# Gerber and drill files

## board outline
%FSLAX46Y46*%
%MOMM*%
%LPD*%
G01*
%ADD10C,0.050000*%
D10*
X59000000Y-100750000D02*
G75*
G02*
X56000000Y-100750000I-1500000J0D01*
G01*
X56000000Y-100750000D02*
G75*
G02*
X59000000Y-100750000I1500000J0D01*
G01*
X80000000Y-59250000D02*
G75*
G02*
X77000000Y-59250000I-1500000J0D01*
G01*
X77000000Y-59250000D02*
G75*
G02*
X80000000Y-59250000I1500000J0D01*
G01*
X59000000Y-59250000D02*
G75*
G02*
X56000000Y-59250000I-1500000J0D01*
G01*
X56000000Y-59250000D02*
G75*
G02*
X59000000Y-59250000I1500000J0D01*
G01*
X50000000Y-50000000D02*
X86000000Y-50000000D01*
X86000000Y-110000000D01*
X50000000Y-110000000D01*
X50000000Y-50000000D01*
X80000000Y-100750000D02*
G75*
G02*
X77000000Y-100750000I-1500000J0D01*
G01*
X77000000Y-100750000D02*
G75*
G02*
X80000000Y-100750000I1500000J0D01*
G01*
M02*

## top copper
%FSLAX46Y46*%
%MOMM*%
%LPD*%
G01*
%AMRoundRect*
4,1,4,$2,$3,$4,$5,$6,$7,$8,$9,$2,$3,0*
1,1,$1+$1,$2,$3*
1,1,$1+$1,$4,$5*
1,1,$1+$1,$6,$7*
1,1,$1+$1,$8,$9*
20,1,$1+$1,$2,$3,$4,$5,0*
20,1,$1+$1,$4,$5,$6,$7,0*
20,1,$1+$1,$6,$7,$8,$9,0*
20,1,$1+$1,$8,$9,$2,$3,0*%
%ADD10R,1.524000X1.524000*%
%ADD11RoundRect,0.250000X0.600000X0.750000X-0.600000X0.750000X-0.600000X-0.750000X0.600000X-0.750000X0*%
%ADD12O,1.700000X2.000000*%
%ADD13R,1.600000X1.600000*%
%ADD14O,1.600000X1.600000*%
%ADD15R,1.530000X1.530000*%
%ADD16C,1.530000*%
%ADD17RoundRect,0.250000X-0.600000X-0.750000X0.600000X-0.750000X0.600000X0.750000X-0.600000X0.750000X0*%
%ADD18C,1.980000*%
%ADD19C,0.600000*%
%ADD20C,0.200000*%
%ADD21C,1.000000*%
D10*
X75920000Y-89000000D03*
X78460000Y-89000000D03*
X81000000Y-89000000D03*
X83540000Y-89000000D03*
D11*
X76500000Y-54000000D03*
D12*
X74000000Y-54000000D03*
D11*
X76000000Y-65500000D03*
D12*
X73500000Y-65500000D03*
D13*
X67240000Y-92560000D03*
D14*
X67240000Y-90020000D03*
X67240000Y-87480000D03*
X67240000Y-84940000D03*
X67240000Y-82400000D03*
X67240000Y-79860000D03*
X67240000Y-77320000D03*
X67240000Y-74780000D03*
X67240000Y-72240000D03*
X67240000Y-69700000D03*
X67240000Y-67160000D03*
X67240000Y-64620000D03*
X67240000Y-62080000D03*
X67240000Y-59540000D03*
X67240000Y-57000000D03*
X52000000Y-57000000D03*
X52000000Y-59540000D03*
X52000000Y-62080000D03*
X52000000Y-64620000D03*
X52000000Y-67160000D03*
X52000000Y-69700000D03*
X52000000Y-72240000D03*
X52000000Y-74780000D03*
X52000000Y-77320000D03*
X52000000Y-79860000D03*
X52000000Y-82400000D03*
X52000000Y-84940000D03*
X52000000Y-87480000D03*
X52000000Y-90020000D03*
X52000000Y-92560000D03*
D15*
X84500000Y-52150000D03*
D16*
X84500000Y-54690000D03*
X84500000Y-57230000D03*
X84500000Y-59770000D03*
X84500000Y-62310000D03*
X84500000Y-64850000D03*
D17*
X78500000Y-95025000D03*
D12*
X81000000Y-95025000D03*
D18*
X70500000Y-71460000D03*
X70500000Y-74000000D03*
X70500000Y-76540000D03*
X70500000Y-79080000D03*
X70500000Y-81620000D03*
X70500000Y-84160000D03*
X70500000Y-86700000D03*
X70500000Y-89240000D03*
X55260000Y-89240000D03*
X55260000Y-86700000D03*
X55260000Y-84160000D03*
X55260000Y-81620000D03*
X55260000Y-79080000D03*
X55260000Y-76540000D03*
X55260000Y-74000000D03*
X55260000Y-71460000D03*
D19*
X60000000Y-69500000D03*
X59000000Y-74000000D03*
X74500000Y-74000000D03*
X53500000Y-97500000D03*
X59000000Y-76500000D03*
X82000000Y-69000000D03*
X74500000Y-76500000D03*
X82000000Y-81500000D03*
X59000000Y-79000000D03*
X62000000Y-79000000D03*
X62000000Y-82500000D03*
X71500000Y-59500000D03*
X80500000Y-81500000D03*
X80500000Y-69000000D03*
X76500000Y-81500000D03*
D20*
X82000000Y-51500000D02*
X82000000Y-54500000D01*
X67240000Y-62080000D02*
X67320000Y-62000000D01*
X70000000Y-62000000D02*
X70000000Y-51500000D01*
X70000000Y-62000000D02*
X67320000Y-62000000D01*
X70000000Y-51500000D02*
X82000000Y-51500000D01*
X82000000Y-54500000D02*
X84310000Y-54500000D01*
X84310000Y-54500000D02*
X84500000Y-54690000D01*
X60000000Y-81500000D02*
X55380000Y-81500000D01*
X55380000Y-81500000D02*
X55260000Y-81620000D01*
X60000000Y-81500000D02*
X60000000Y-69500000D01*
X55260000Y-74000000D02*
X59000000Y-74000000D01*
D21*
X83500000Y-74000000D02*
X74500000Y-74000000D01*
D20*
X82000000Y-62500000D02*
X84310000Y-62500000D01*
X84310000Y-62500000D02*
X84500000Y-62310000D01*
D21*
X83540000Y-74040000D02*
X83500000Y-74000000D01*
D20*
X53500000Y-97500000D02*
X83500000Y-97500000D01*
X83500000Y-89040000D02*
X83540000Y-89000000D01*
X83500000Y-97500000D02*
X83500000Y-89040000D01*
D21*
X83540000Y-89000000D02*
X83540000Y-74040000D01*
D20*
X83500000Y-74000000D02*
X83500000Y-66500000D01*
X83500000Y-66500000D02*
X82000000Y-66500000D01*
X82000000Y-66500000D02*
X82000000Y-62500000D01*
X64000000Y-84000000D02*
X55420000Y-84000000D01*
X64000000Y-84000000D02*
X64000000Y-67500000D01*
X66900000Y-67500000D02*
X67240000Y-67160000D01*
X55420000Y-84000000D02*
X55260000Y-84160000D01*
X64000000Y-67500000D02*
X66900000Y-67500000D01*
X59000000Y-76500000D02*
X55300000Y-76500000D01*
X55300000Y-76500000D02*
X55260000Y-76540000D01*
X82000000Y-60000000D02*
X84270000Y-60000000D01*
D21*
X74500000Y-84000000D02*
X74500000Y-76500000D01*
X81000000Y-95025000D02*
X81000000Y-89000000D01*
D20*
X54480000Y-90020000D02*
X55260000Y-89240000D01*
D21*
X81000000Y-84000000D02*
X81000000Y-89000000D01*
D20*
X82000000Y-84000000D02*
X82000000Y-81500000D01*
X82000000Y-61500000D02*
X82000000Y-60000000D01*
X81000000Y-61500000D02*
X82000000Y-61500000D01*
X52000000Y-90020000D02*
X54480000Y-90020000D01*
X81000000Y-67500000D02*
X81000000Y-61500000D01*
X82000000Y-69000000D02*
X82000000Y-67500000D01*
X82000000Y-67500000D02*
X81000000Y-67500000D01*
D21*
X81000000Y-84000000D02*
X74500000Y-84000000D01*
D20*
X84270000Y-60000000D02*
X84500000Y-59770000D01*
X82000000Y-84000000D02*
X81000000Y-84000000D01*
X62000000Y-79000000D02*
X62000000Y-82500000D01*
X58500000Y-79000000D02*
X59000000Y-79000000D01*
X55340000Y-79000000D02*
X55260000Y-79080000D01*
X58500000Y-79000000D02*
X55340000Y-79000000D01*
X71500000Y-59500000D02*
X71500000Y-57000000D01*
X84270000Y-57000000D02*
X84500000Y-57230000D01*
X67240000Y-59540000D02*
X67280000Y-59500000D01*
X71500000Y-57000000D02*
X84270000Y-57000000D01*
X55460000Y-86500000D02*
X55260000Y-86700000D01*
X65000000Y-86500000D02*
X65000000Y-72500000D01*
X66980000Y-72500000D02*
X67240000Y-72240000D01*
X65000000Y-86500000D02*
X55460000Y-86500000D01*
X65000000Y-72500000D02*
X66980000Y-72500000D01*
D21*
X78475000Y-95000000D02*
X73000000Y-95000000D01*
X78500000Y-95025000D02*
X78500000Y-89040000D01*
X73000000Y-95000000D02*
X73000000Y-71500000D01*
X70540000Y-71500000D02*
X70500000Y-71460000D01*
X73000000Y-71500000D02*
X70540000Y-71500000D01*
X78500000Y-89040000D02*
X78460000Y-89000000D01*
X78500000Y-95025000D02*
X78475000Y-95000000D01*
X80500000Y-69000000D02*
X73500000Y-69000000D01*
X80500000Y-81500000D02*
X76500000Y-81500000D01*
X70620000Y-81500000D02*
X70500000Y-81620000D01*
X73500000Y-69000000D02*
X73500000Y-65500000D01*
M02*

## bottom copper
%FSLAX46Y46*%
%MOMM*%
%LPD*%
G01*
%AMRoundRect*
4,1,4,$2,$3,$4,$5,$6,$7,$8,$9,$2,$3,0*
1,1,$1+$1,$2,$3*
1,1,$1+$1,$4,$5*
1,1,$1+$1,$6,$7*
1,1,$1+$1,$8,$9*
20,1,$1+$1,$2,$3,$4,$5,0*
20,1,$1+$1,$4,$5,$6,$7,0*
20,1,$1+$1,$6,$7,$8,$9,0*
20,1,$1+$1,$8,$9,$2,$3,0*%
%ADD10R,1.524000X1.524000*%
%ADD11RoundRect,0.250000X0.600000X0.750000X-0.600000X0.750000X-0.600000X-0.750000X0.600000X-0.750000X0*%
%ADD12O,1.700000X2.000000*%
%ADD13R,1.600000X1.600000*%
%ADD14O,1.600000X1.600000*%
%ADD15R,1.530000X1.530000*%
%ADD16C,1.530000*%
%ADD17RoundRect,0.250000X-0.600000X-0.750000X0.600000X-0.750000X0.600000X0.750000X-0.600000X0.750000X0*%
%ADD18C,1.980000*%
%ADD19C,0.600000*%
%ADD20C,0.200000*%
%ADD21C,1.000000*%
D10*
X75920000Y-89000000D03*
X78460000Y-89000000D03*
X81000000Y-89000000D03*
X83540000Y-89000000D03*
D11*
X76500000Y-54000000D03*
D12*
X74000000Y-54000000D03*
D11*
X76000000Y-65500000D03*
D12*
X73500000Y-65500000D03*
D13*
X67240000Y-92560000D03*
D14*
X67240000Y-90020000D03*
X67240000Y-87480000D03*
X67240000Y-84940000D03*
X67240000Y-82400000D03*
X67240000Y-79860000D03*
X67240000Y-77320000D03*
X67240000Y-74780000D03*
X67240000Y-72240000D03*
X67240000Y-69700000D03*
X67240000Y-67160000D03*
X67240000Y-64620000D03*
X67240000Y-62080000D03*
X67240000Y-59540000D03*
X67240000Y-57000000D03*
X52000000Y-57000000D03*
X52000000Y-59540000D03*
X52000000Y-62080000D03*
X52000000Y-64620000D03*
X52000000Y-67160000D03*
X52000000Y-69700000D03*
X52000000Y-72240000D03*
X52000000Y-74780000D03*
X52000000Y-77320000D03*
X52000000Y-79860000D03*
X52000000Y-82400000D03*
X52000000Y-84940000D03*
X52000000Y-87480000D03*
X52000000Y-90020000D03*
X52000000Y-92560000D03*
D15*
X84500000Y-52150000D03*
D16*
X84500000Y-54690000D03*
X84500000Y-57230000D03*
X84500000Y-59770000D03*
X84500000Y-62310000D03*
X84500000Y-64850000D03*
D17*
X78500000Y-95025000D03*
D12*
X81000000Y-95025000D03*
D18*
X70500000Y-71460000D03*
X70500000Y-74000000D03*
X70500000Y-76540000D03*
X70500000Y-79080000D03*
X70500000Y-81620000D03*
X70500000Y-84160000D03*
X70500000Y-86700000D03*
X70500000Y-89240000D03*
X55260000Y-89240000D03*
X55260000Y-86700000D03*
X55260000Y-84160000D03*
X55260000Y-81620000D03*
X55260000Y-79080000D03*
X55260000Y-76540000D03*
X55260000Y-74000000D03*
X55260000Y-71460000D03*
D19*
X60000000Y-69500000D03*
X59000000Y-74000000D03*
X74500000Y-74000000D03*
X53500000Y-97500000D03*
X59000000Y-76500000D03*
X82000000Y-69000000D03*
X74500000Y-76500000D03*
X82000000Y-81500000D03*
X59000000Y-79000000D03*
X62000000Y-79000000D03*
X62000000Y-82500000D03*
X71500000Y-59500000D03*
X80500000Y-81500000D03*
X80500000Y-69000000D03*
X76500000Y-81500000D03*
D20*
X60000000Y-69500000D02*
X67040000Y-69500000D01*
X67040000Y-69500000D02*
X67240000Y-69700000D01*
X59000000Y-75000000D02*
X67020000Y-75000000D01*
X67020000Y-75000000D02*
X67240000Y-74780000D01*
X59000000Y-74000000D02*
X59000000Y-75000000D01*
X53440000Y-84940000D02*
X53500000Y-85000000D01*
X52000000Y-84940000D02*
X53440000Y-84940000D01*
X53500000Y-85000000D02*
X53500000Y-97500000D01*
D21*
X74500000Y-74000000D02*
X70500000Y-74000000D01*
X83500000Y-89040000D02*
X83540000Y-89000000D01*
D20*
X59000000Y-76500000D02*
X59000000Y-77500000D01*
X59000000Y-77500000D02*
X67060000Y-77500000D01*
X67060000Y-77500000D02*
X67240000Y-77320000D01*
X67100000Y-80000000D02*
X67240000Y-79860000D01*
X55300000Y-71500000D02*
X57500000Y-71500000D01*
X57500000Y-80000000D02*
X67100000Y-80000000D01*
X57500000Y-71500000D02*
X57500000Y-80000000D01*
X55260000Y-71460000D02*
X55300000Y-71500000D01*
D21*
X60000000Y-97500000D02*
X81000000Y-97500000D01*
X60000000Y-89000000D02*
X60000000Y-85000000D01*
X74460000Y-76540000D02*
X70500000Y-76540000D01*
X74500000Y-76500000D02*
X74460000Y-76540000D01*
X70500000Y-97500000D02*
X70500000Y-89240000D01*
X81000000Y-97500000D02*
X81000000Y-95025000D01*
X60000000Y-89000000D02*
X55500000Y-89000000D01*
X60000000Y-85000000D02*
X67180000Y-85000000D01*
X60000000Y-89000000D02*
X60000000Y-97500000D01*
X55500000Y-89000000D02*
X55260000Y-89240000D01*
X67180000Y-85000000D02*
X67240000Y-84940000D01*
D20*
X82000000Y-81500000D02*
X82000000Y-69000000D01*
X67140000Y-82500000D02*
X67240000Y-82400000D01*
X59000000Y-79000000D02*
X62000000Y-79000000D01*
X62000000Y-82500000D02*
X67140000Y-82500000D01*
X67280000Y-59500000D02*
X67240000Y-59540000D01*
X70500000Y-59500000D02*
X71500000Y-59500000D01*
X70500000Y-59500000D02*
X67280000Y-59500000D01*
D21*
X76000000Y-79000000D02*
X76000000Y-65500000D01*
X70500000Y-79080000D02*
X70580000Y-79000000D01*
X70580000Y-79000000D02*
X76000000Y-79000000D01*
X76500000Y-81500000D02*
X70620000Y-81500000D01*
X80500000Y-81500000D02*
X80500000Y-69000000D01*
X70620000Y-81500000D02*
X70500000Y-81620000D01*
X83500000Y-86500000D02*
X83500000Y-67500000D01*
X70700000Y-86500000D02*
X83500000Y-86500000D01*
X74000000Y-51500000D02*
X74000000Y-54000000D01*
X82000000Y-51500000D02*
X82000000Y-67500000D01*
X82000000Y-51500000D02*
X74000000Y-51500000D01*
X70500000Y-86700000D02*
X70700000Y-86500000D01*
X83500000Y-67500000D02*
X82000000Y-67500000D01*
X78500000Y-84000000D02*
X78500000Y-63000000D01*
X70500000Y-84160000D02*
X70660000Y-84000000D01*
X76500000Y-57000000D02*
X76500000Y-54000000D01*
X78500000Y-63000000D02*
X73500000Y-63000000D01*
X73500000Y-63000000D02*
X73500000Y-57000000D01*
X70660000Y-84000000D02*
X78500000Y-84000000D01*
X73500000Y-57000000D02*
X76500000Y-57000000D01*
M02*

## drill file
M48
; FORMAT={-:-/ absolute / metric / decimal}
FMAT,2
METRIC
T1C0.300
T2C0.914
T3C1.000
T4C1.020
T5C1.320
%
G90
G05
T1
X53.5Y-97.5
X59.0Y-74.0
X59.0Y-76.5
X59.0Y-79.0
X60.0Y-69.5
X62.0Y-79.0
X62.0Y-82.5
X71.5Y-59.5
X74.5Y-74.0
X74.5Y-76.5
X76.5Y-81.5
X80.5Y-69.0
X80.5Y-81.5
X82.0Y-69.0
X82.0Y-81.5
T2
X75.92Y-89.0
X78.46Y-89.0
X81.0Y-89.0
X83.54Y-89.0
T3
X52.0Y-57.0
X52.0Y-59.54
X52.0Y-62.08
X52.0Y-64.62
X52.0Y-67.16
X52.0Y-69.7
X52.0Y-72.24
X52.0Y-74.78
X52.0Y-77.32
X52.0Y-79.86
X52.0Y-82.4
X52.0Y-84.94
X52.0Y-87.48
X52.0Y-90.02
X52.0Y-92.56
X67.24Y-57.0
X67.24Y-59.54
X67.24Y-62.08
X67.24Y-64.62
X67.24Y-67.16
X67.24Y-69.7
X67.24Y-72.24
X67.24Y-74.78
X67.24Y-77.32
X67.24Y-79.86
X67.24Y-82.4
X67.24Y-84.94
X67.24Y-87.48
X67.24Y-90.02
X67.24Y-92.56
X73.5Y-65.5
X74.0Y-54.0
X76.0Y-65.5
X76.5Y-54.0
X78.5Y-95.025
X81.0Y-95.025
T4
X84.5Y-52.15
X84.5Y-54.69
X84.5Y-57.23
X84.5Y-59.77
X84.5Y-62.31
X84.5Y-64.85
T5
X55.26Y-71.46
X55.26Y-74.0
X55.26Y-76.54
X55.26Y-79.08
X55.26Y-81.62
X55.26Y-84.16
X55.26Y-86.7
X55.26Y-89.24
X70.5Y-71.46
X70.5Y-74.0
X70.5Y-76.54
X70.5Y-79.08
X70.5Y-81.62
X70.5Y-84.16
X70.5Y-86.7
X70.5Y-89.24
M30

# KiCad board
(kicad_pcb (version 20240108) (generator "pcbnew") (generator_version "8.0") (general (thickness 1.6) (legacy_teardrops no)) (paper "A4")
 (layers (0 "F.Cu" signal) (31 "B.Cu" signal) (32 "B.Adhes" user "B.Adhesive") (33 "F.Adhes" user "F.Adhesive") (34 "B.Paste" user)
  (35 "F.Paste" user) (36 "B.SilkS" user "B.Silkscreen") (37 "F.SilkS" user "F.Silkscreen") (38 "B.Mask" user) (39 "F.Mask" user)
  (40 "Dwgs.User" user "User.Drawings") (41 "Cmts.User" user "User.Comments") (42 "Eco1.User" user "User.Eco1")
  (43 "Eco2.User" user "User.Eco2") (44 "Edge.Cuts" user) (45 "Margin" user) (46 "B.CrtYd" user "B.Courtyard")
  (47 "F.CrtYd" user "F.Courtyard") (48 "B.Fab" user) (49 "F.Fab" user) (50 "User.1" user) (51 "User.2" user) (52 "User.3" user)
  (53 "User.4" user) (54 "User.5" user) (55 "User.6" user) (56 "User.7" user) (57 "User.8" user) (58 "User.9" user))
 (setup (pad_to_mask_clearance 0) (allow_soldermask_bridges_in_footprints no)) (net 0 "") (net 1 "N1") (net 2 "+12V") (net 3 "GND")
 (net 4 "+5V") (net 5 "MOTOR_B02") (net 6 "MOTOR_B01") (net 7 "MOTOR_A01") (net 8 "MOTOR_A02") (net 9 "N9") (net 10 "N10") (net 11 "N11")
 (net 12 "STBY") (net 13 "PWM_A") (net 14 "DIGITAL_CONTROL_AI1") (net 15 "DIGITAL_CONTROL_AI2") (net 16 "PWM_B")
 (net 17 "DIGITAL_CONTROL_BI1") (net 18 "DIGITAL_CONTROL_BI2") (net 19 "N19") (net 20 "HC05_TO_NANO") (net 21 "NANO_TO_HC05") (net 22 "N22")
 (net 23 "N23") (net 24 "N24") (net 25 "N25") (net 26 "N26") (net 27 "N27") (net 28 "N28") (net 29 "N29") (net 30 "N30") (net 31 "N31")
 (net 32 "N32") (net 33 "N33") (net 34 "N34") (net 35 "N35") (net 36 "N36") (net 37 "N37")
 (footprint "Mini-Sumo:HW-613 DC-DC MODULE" (layer "F.Cu") (at 75.92 89 90)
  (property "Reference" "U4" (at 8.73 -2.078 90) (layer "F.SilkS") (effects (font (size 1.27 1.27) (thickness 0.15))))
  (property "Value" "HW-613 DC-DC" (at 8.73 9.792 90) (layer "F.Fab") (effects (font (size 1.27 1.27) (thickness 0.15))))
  (pad "1" thru_hole rect (at 0 0 90) (size 1.524 1.524) (drill 0.9144) (layers "*.Cu" "*.Mask") (remove_unused_layers no) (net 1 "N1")
   (solder_mask_margin 0.0508) (thermal_bridge_angle 0))
  (pad "2" thru_hole rect (at 0 2.54 90) (size 1.524 1.524) (drill 0.9144) (layers "*.Cu" "*.Mask") (remove_unused_layers no) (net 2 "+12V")
   (solder_mask_margin 0.0508) (thermal_bridge_angle 0))
  (pad "3" thru_hole rect (at 0 5.08 90) (size 1.524 1.524) (drill 0.9144) (layers "*.Cu" "*.Mask") (remove_unused_layers no) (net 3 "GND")
   (solder_mask_margin 0.0508) (thermal_bridge_angle 0))
  (pad "4" thru_hole rect (at 0 7.62 90) (size 1.524 1.524) (drill 0.9144) (layers "*.Cu" "*.Mask") (remove_unused_layers no) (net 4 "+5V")
   (solder_mask_margin 0.0508) (thermal_bridge_angle 0)))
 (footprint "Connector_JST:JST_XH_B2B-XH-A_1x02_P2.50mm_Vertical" (layer "F.Cu") (at 76.5 54 180)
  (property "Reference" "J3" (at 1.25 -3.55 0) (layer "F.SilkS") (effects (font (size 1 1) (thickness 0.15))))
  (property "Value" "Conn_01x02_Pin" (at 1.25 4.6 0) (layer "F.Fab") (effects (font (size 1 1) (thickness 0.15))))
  (pad "1" thru_hole roundrect (at 0 0 180) (size 1.7 2) (drill 1) (layers "*.Cu" "*.Mask") (remove_unused_layers no)
   (roundrect_rratio 0.147059) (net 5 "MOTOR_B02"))
  (pad "2" thru_hole oval (at 2.5 0 180) (size 1.7 2) (drill 1) (layers "*.Cu" "*.Mask") (remove_unused_layers no) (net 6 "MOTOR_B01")))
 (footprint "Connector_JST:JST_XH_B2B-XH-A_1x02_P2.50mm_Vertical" (layer "F.Cu") (at 76 65.5 180)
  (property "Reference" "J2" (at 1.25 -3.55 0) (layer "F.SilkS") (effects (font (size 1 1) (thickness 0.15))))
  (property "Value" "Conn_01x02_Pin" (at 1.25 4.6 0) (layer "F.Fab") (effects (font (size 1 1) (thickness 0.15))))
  (pad "1" thru_hole roundrect (at 0 0 180) (size 1.7 2) (drill 1) (layers "*.Cu" "*.Mask") (remove_unused_layers no)
   (roundrect_rratio 0.147059) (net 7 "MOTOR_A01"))
  (pad "2" thru_hole oval (at 2.5 0 180) (size 1.7 2) (drill 1) (layers "*.Cu" "*.Mask") (remove_unused_layers no) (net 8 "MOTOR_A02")))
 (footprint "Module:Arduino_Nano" (layer "F.Cu") (at 67.24 92.56 180)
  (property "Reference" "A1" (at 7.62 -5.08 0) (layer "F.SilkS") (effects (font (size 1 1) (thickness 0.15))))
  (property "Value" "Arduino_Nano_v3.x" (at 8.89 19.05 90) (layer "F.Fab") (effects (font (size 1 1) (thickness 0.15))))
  (pad "1" thru_hole rect (at 0 0 180) (size 1.6 1.6) (drill 1) (layers "*.Cu" "*.Mask") (remove_unused_layers no) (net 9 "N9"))
  (pad "2" thru_hole oval (at 0 2.54 180) (size 1.6 1.6) (drill 1) (layers "*.Cu" "*.Mask") (remove_unused_layers no) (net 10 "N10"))
  (pad "3" thru_hole oval (at 0 5.08 180) (size 1.6 1.6) (drill 1) (layers "*.Cu" "*.Mask") (remove_unused_layers no) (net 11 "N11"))
  (pad "4" thru_hole oval (at 0 7.62 180) (size 1.6 1.6) (drill 1) (layers "*.Cu" "*.Mask") (remove_unused_layers no) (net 3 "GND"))
  (pad "5" thru_hole oval (at 0 10.16 180) (size 1.6 1.6) (drill 1) (layers "*.Cu" "*.Mask") (remove_unused_layers no) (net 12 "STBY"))
  (pad "6" thru_hole oval (at 0 12.7 180) (size 1.6 1.6) (drill 1) (layers "*.Cu" "*.Mask") (remove_unused_layers no) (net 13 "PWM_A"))
  (pad "7" thru_hole oval (at 0 15.24 180) (size 1.6 1.6) (drill 1) (layers "*.Cu" "*.Mask") (remove_unused_layers no)
   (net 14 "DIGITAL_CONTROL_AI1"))
  (pad "8" thru_hole oval (at 0 17.78 180) (size 1.6 1.6) (drill 1) (layers "*.Cu" "*.Mask") (remove_unused_layers no)
   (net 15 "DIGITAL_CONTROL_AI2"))
  (pad "9" thru_hole oval (at 0 20.32 180) (size 1.6 1.6) (drill 1) (layers "*.Cu" "*.Mask") (remove_unused_layers no) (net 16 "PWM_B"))
  (pad "10" thru_hole oval (at 0 22.86 180) (size 1.6 1.6) (drill 1) (layers "*.Cu" "*.Mask") (remove_unused_layers no)
   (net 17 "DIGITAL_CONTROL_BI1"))
  (pad "11" thru_hole oval (at 0 25.4 180) (size 1.6 1.6) (drill 1) (layers "*.Cu" "*.Mask") (remove_unused_layers no)
   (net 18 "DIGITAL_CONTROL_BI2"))
  (pad "12" thru_hole oval (at 0 27.94 180) (size 1.6 1.6) (drill 1) (layers "*.Cu" "*.Mask") (remove_unused_layers no) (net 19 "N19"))
  (pad "13" thru_hole oval (at 0 30.48 180) (size 1.6 1.6) (drill 1) (layers "*.Cu" "*.Mask") (remove_unused_layers no)
   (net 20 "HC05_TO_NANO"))
  (pad "14" thru_hole oval (at 0 33.02 180) (size 1.6 1.6) (drill 1) (layers "*.Cu" "*.Mask") (remove_unused_layers no)
   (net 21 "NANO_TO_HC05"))
  (pad "15" thru_hole oval (at 0 35.56 180) (size 1.6 1.6) (drill 1) (layers "*.Cu" "*.Mask") (remove_unused_layers no) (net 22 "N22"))
  (pad "16" thru_hole oval (at 15.24 35.56 180) (size 1.6 1.6) (drill 1) (layers "*.Cu" "*.Mask") (remove_unused_layers no) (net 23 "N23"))
  (pad "17" thru_hole oval (at 15.24 33.02 180) (size 1.6 1.6) (drill 1) (layers "*.Cu" "*.Mask") (remove_unused_layers no) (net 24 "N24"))
  (pad "18" thru_hole oval (at 15.24 30.48 180) (size 1.6 1.6) (drill 1) (layers "*.Cu" "*.Mask") (remove_unused_layers no) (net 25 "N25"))
  (pad "19" thru_hole oval (at 15.24 27.94 180) (size 1.6 1.6) (drill 1) (layers "*.Cu" "*.Mask") (remove_unused_layers no) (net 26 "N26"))
  (pad "20" thru_hole oval (at 15.24 25.4 180) (size 1.6 1.6) (drill 1) (layers "*.Cu" "*.Mask") (remove_unused_layers no) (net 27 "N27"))
  (pad "21" thru_hole oval (at 15.24 22.86 180) (size 1.6 1.6) (drill 1) (layers "*.Cu" "*.Mask") (remove_unused_layers no) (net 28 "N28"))
  (pad "22" thru_hole oval (at 15.24 20.32 180) (size 1.6 1.6) (drill 1) (layers "*.Cu" "*.Mask") (remove_unused_layers no) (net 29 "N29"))
  (pad "23" thru_hole oval (at 15.24 17.78 180) (size 1.6 1.6) (drill 1) (layers "*.Cu" "*.Mask") (remove_unused_layers no) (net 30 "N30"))
  (pad "24" thru_hole oval (at 15.24 15.24 180) (size 1.6 1.6) (drill 1) (layers "*.Cu" "*.Mask") (remove_unused_layers no) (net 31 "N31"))
  (pad "25" thru_hole oval (at 15.24 12.7 180) (size 1.6 1.6) (drill 1) (layers "*.Cu" "*.Mask") (remove_unused_layers no) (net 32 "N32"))
  (pad "26" thru_hole oval (at 15.24 10.16 180) (size 1.6 1.6) (drill 1) (layers "*.Cu" "*.Mask") (remove_unused_layers no) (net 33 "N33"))
  (pad "27" thru_hole oval (at 15.24 7.62 180) (size 1.6 1.6) (drill 1) (layers "*.Cu" "*.Mask") (remove_unused_layers no) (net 4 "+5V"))
  (pad "28" thru_hole oval (at 15.24 5.08 180) (size 1.6 1.6) (drill 1) (layers "*.Cu" "*.Mask") (remove_unused_layers no) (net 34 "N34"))
  (pad "29" thru_hole oval (at 15.24 2.54 180) (size 1.6 1.6) (drill 1) (layers "*.Cu" "*.Mask") (remove_unused_layers no) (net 3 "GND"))
  (pad "30" thru_hole oval (at 15.24 0 180) (size 1.6 1.6) (drill 1) (layers "*.Cu" "*.Mask") (remove_unused_layers no) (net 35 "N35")))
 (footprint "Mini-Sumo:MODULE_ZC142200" (layer "F.Cu") (at 84.5 58.5)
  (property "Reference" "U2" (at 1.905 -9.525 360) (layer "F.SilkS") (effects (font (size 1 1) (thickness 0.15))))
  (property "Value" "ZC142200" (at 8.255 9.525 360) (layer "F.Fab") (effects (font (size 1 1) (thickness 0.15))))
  (pad "1" thru_hole rect (at 0 -6.35) (size 1.53 1.53) (drill 1.02) (layers "*.Cu" "*.Mask") (remove_unused_layers no) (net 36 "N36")
   (solder_mask_margin 0.102))
  (pad "2" thru_hole circle (at 0 -3.81) (size 1.53 1.53) (drill 1.02) (layers "*.Cu" "*.Mask") (remove_unused_layers no)
   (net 20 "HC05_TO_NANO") (solder_mask_margin 0.102))
  (pad "3" thru_hole circle (at 0 -1.27) (size 1.53 1.53) (drill 1.02) (layers "*.Cu" "*.Mask") (remove_unused_layers no)
   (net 21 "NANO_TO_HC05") (solder_mask_margin 0.102))
  (pad "4" thru_hole circle (at 0 1.27) (size 1.53 1.53) (drill 1.02) (layers "*.Cu" "*.Mask") (remove_unused_layers no) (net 3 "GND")
   (solder_mask_margin 0.102))
  (pad "5" thru_hole circle (at 0 3.81) (size 1.53 1.53) (drill 1.02) (layers "*.Cu" "*.Mask") (remove_unused_layers no) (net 4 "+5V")
   (solder_mask_margin 0.102))
  (pad "6" thru_hole circle (at 0 6.35) (size 1.53 1.53) (drill 1.02) (layers "*.Cu" "*.Mask") (remove_unused_layers no) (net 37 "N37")
   (solder_mask_margin 0.102)))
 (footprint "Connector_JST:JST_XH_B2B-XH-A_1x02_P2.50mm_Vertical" (layer "F.Cu") (at 78.5 95.025)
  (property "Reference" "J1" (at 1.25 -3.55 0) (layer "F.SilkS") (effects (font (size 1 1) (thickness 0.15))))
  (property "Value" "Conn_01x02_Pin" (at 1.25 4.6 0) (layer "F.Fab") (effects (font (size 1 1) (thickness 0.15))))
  (pad "1" thru_hole roundrect (at 0 0) (size 1.7 2) (drill 1) (layers "*.Cu" "*.Mask") (remove_unused_layers no)
   (roundrect_rratio 0.147059) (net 2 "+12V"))
  (pad "2" thru_hole oval (at 2.5 0) (size 1.7 2) (drill 1) (layers "*.Cu" "*.Mask") (remove_unused_layers no) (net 3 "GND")))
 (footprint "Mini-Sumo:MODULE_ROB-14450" (layer "B.Cu") (at 62.88 80.35 180)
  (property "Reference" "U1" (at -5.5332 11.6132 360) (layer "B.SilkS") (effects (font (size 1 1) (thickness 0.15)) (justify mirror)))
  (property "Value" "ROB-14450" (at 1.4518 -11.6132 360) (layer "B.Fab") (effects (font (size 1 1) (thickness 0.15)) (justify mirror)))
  (pad "1" thru_hole circle (at -7.62 8.89 180) (size 1.98 1.98) (drill 1.32) (layers "*.Cu" "*.Mask") (remove_unused_layers no)
   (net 2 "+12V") (solder_mask_margin 0.102))
  (pad "2" thru_hole circle (at -7.62 6.35 180) (size 1.98 1.98) (drill 1.32) (layers "*.Cu" "*.Mask") (remove_unused_layers no)
   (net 4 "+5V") (solder_mask_margin 0.102))
  (pad "3" thru_hole circle (at -7.62 3.81 180) (size 1.98 1.98) (drill 1.32) (layers "*.Cu" "*.Mask") (remove_unused_layers no)
   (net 3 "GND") (solder_mask_margin 0.102))
  (pad "4" thru_hole circle (at -7.62 1.27 180) (size 1.98 1.98) (drill 1.32) (layers "*.Cu" "*.Mask") (remove_unused_layers no)
   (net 7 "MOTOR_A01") (solder_mask_margin 0.102))
  (pad "5" thru_hole circle (at -7.62 -1.27 180) (size 1.98 1.98) (drill 1.32) (layers "*.Cu" "*.Mask") (remove_unused_layers no)
   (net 8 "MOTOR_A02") (solder_mask_margin 0.102))
  (pad "6" thru_hole circle (at -7.62 -3.81 180) (size 1.98 1.98) (drill 1.32) (layers "*.Cu" "*.Mask") (remove_unused_layers no)
   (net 5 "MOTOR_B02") (solder_mask_margin 0.102))
  (pad "7" thru_hole circle (at -7.62 -6.35 180) (size 1.98 1.98) (drill 1.32) (layers "*.Cu" "*.Mask") (remove_unused_layers no)
   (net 6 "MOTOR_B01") (solder_mask_margin 0.102))
  (pad "8" thru_hole circle (at -7.62 -8.89 180) (size 1.98 1.98) (drill 1.32) (layers "*.Cu" "*.Mask") (remove_unused_layers no)
   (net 3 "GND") (solder_mask_margin 0.102))
  (pad "9" thru_hole circle (at 7.62 -8.89 180) (size 1.98 1.98) (drill 1.32) (layers "*.Cu" "*.Mask") (remove_unused_layers no)
   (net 3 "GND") (solder_mask_margin 0.102))
  (pad "10" thru_hole circle (at 7.62 -6.35 180) (size 1.98 1.98) (drill 1.32) (layers "*.Cu" "*.Mask") (remove_unused_layers no)
   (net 16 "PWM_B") (solder_mask_margin 0.102))
  (pad "11" thru_hole circle (at 7.62 -3.81 180) (size 1.98 1.98) (drill 1.32) (layers "*.Cu" "*.Mask") (remove_unused_layers no)
   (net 18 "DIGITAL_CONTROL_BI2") (solder_mask_margin 0.102))
  (pad "12" thru_hole circle (at 7.62 -1.27 180) (size 1.98 1.98) (drill 1.32) (layers "*.Cu" "*.Mask") (remove_unused_layers no)
   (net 17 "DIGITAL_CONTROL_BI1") (solder_mask_margin 0.102))
  (pad "13" thru_hole circle (at 7.62 1.27 180) (size 1.98 1.98) (drill 1.32) (layers "*.Cu" "*.Mask") (remove_unused_layers no)
   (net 12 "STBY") (solder_mask_margin 0.102))
  (pad "14" thru_hole circle (at 7.62 3.81 180) (size 1.98 1.98) (drill 1.32) (layers "*.Cu" "*.Mask") (remove_unused_layers no)
   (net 14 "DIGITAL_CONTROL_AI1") (solder_mask_margin 0.102))
  (pad "15" thru_hole circle (at 7.62 6.35 180) (size 1.98 1.98) (drill 1.32) (layers "*.Cu" "*.Mask") (remove_unused_layers no)
   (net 15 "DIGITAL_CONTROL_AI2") (solder_mask_margin 0.102))
  (pad "16" thru_hole circle (at 7.62 8.89 180) (size 1.98 1.98) (drill 1.32) (layers "*.Cu" "*.Mask") (remove_unused_layers no)
   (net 13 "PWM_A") (solder_mask_margin 0.102)))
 (gr_circle (center 57.5 100.75) (end 59 100.75) (stroke (width 0.05) (type default)) (fill none) (layer "Edge.Cuts"))
 (gr_circle (center 78.5 59.25) (end 80 59.25) (stroke (width 0.05) (type default)) (fill none) (layer "Edge.Cuts"))
 (gr_circle (center 57.5 59.25) (end 59 59.25) (stroke (width 0.05) (type default)) (fill none) (layer "Edge.Cuts"))
 (gr_rect (start 50 50) (end 86 110) (stroke (width 0.05) (type default)) (fill none) (layer "Edge.Cuts"))
 (gr_circle (center 78.5 100.75) (end 80 100.75) (stroke (width 0.05) (type default)) (fill none) (layer "Edge.Cuts"))
 (segment (start 82 51.5) (end 82 54.5) (width 0.2) (layer "F.Cu") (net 20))
 (segment (start 67.24 62.08) (end 67.32 62) (width 0.2) (layer "F.Cu") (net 20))
 (segment (start 70 62) (end 70 51.5) (width 0.2) (layer "F.Cu") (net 20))
 (segment (start 70 62) (end 67.32 62) (width 0.2) (layer "F.Cu") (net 20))
 (segment (start 70 51.5) (end 82 51.5) (width 0.2) (layer "F.Cu") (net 20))
 (segment (start 82 54.5) (end 84.31 54.5) (width 0.2) (layer "F.Cu") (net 20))
 (segment (start 84.31 54.5) (end 84.5 54.69) (width 0.2) (layer "F.Cu") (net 20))
 (segment (start 60 81.5) (end 55.38 81.5) (width 0.2) (layer "F.Cu") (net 17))
 (segment (start 55.38 81.5) (end 55.26 81.62) (width 0.2) (layer "F.Cu") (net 17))
 (segment (start 60 81.5) (end 60 69.5) (width 0.2) (layer "F.Cu") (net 17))
 (via (at 60 69.5) (size 0.6) (drill 0.3) (layers "F.Cu" "B.Cu") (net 17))
 (segment (start 60 69.5) (end 67.04 69.5) (width 0.2) (layer "B.Cu") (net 17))
 (segment (start 67.04 69.5) (end 67.24 69.7) (width 0.2) (layer "B.Cu") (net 17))
 (segment (start 55.26 74) (end 59 74) (width 0.2) (layer "F.Cu") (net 15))
 (via (at 59 74) (size 0.6) (drill 0.3) (layers "F.Cu" "B.Cu") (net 15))
 (segment (start 59 75) (end 67.02 75) (width 0.2) (layer "B.Cu") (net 15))
 (segment (start 67.02 75) (end 67.24 74.78) (width 0.2) (layer "B.Cu") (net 15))
 (segment (start 59 74) (end 59 75) (width 0.2) (layer "B.Cu") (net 15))
 (segment (start 83.5 74) (end 74.5 74) (width 1) (layer "F.Cu") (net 4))
 (segment (start 82 62.5) (end 84.31 62.5) (width 0.2) (layer "F.Cu") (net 4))
 (segment (start 84.31 62.5) (end 84.5 62.31) (width 0.2) (layer "F.Cu") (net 4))
 (segment (start 83.54 74.04) (end 83.5 74) (width 1) (layer "F.Cu") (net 4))
 (segment (start 53.5 97.5) (end 83.5 97.5) (width 0.2) (layer "F.Cu") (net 4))
 (segment (start 83.5 89.04) (end 83.54 89) (width 0.2) (layer "F.Cu") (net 4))
 (segment (start 83.5 97.5) (end 83.5 89.04) (width 0.2) (layer "F.Cu") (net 4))
 (segment (start 83.54 89) (end 83.54 74.04) (width 1) (layer "F.Cu") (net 4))
 (segment (start 83.5 74) (end 83.5 66.5) (width 0.2) (layer "F.Cu") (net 4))
 (segment (start 83.5 66.5) (end 82 66.5) (width 0.2) (layer "F.Cu") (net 4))
 (segment (start 82 66.5) (end 82 62.5) (width 0.2) (layer "F.Cu") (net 4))
 (via (at 74.5 74) (size 0.6) (drill 0.3) (layers "F.Cu" "B.Cu") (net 4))
 (via (at 53.5 97.5) (size 0.6) (drill 0.3) (layers "F.Cu" "B.Cu") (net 4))
 (segment (start 53.44 84.94) (end 53.5 85) (width 0.2) (layer "B.Cu") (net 4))
 (segment (start 52 84.94) (end 53.44 84.94) (width 0.2) (layer "B.Cu") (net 4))
 (segment (start 53.5 85) (end 53.5 97.5) (width 0.2) (layer "B.Cu") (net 4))
 (segment (start 74.5 74) (end 70.5 74) (width 1) (layer "B.Cu") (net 4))
 (segment (start 83.5 89.04) (end 83.54 89) (width 1) (layer "B.Cu") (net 4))
 (segment (start 64 84) (end 55.42 84) (width 0.2) (layer "F.Cu") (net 18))
 (segment (start 64 84) (end 64 67.5) (width 0.2) (layer "F.Cu") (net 18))
 (segment (start 66.9 67.5) (end 67.24 67.16) (width 0.2) (layer "F.Cu") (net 18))
 (segment (start 55.42 84) (end 55.26 84.16) (width 0.2) (layer "F.Cu") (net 18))
 (segment (start 64 67.5) (end 66.9 67.5) (width 0.2) (layer "F.Cu") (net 18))
 (segment (start 59 76.5) (end 55.3 76.5) (width 0.2) (layer "F.Cu") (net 14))
 (segment (start 55.3 76.5) (end 55.26 76.54) (width 0.2) (layer "F.Cu") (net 14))
 (via (at 59 76.5) (size 0.6) (drill 0.3) (layers "F.Cu" "B.Cu") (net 14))
 (segment (start 59 76.5) (end 59 77.5) (width 0.2) (layer "B.Cu") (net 14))
 (segment (start 59 77.5) (end 67.06 77.5) (width 0.2) (layer "B.Cu") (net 14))
 (segment (start 67.06 77.5) (end 67.24 77.32) (width 0.2) (layer "B.Cu") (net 14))
 (segment (start 67.1 80) (end 67.24 79.86) (width 0.2) (layer "B.Cu") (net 13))
 (segment (start 55.3 71.5) (end 57.5 71.5) (width 0.2) (layer "B.Cu") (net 13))
 (segment (start 57.5 80) (end 67.1 80) (width 0.2) (layer "B.Cu") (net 13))
 (segment (start 57.5 71.5) (end 57.5 80) (width 0.2) (layer "B.Cu") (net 13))
 (segment (start 55.26 71.46) (end 55.3 71.5) (width 0.2) (layer "B.Cu") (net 13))
 (segment (start 82 60) (end 84.27 60) (width 0.2) (layer "F.Cu") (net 3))
 (segment (start 74.5 84) (end 74.5 76.5) (width 1) (layer "F.Cu") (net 3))
 (segment (start 81 95.025) (end 81 89) (width 1) (layer "F.Cu") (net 3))
 (segment (start 54.48 90.02) (end 55.26 89.24) (width 0.2) (layer "F.Cu") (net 3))
 (segment (start 81 84) (end 81 89) (width 1) (layer "F.Cu") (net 3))
 (segment (start 82 84) (end 82 81.5) (width 0.2) (layer "F.Cu") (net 3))
 (segment (start 82 61.5) (end 82 60) (width 0.2) (layer "F.Cu") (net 3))
 (segment (start 81 61.5) (end 82 61.5) (width 0.2) (layer "F.Cu") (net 3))
 (segment (start 52 90.02) (end 54.48 90.02) (width 0.2) (layer "F.Cu") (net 3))
 (segment (start 81 67.5) (end 81 61.5) (width 0.2) (layer "F.Cu") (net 3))
 (segment (start 82 69) (end 82 67.5) (width 0.2) (layer "F.Cu") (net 3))
 (segment (start 82 67.5) (end 81 67.5) (width 0.2) (layer "F.Cu") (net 3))
 (segment (start 81 84) (end 74.5 84) (width 1) (layer "F.Cu") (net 3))
 (segment (start 84.27 60) (end 84.5 59.77) (width 0.2) (layer "F.Cu") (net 3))
 (segment (start 82 84) (end 81 84) (width 0.2) (layer "F.Cu") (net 3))
 (via (at 82 69) (size 0.6) (drill 0.3) (layers "F.Cu" "B.Cu") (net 3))
 (via (at 74.5 76.5) (size 0.6) (drill 0.3) (layers "F.Cu" "B.Cu") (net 3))
 (via (at 82 81.5) (size 0.6) (drill 0.3) (layers "F.Cu" "B.Cu") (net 3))
 (segment (start 60 97.5) (end 81 97.5) (width 1) (layer "B.Cu") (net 3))
 (segment (start 60 89) (end 60 85) (width 1) (layer "B.Cu") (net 3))
 (segment (start 74.46 76.54) (end 70.5 76.54) (width 1) (layer "B.Cu") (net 3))
 (segment (start 74.5 76.5) (end 74.46 76.54) (width 1) (layer "B.Cu") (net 3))
 (segment (start 70.5 97.5) (end 70.5 89.24) (width 1) (layer "B.Cu") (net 3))
 (segment (start 81 97.5) (end 81 95.025) (width 1) (layer "B.Cu") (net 3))
 (segment (start 60 89) (end 55.5 89) (width 1) (layer "B.Cu") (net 3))
 (segment (start 60 85) (end 67.18 85) (width 1) (layer "B.Cu") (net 3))
 (segment (start 60 89) (end 60 97.5) (width 1) (layer "B.Cu") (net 3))
 (segment (start 55.5 89) (end 55.26 89.24) (width 1) (layer "B.Cu") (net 3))
 (segment (start 67.18 85) (end 67.24 84.94) (width 1) (layer "B.Cu") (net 3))
 (segment (start 82 81.5) (end 82 69) (width 0.2) (layer "B.Cu") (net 3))
 (segment (start 62 79) (end 62 82.5) (width 0.2) (layer "F.Cu") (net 12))
 (segment (start 58.5 79) (end 59 79) (width 0.2) (layer "F.Cu") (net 12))
 (segment (start 55.34 79) (end 55.26 79.08) (width 0.2) (layer "F.Cu") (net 12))
 (segment (start 58.5 79) (end 55.34 79) (width 0.2) (layer "F.Cu") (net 12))
 (via (at 59 79) (size 0.6) (drill 0.3) (layers "F.Cu" "B.Cu") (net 12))
 (via (at 62 79) (size 0.6) (drill 0.3) (layers "F.Cu" "B.Cu") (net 12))
 (via (at 62 82.5) (size 0.6) (drill 0.3) (layers "F.Cu" "B.Cu") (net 12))
 (segment (start 67.14 82.5) (end 67.24 82.4) (width 0.2) (layer "B.Cu") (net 12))
 (segment (start 59 79) (end 62 79) (width 0.2) (layer "B.Cu") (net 12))
 (segment (start 62 82.5) (end 67.14 82.5) (width 0.2) (layer "B.Cu") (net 12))
 (segment (start 71.5 59.5) (end 71.5 57) (width 0.2) (layer "F.Cu") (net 21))
 (segment (start 84.27 57) (end 84.5 57.23) (width 0.2) (layer "F.Cu") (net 21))
 (segment (start 67.24 59.54) (end 67.28 59.5) (width 0.2) (layer "F.Cu") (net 21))
 (segment (start 71.5 57) (end 84.27 57) (width 0.2) (layer "F.Cu") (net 21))
 (via (at 71.5 59.5) (size 0.6) (drill 0.3) (layers "F.Cu" "B.Cu") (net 21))
 (segment (start 67.28 59.5) (end 67.24 59.54) (width 0.2) (layer "B.Cu") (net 21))
 (segment (start 70.5 59.5) (end 71.5 59.5) (width 0.2) (layer "B.Cu") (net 21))
 (segment (start 70.5 59.5) (end 67.28 59.5) (width 0.2) (layer "B.Cu") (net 21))
 (segment (start 55.46 86.5) (end 55.26 86.7) (width 0.2) (layer "F.Cu") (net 16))
 (segment (start 65 86.5) (end 65 72.5) (width 0.2) (layer "F.Cu") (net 16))
 (segment (start 66.98 72.5) (end 67.24 72.24) (width 0.2) (layer "F.Cu") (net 16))
 (segment (start 65 86.5) (end 55.46 86.5) (width 0.2) (layer "F.Cu") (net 16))
 (segment (start 65 72.5) (end 66.98 72.5) (width 0.2) (layer "F.Cu") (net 16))
 (segment (start 78.475 95) (end 73 95) (width 1) (layer "F.Cu") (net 2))
 (segment (start 78.5 95.025) (end 78.5 89.04) (width 1) (layer "F.Cu") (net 2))
 (segment (start 73 95) (end 73 71.5) (width 1) (layer "F.Cu") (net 2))
 (segment (start 70.54 71.5) (end 70.5 71.46) (width 1) (layer "F.Cu") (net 2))
 (segment (start 73 71.5) (end 70.54 71.5) (width 1) (layer "F.Cu") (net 2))
 (segment (start 78.5 89.04) (end 78.46 89) (width 1) (layer "F.Cu") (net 2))
 (segment (start 78.5 95.025) (end 78.475 95) (width 1) (layer "F.Cu") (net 2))
 (segment (start 76 79) (end 76 65.5) (width 1) (layer "B.Cu") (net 7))
 (segment (start 70.5 79.08) (end 70.58 79) (width 1) (layer "B.Cu") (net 7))
 (segment (start 70.58 79) (end 76 79) (width 1) (layer "B.Cu") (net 7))
 (segment (start 80.5 69) (end 73.5 69) (width 1) (layer "F.Cu") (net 8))
 (segment (start 80.5 81.5) (end 76.5 81.5) (width 1) (layer "F.Cu") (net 8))
 (segment (start 70.62 81.5) (end 70.5 81.62) (width 1) (layer "F.Cu") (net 8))
 (segment (start 73.5 69) (end 73.5 65.5) (width 1) (layer "F.Cu") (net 8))
 (via (at 80.5 81.5) (size 0.6) (drill 0.3) (layers "F.Cu" "B.Cu") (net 8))
 (via (at 80.5 69) (size 0.6) (drill 0.3) (layers "F.Cu" "B.Cu") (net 8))
 (via (at 76.5 81.5) (size 0.6) (drill 0.3) (layers "F.Cu" "B.Cu") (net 8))
 (segment (start 76.5 81.5) (end 70.62 81.5) (width 1) (layer "B.Cu") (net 8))
 (segment (start 80.5 81.5) (end 80.5 69) (width 1) (layer "B.Cu") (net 8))
 (segment (start 70.62 81.5) (end 70.5 81.62) (width 1) (layer "B.Cu") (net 8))
 (segment (start 83.5 86.5) (end 83.5 67.5) (width 1) (layer "B.Cu") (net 6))
 (segment (start 70.7 86.5) (end 83.5 86.5) (width 1) (layer "B.Cu") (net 6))
 (segment (start 74 51.5) (end 74 54) (width 1) (layer "B.Cu") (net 6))
 (segment (start 82 51.5) (end 82 67.5) (width 1) (layer "B.Cu") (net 6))
 (segment (start 82 51.5) (end 74 51.5) (width 1) (layer "B.Cu") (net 6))
 (segment (start 70.5 86.7) (end 70.7 86.5) (width 1) (layer "B.Cu") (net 6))
 (segment (start 83.5 67.5) (end 82 67.5) (width 1) (layer "B.Cu") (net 6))
 (segment (start 78.5 84) (end 78.5 63) (width 1) (layer "B.Cu") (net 5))
 (segment (start 70.5 84.16) (end 70.66 84) (width 1) (layer "B.Cu") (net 5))
 (segment (start 76.5 57) (end 76.5 54) (width 1) (layer "B.Cu") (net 5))
 (segment (start 78.5 63) (end 73.5 63) (width 1) (layer "B.Cu") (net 5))
 (segment (start 73.5 63) (end 73.5 57) (width 1) (layer "B.Cu") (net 5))
 (segment (start 70.66 84) (end 78.5 84) (width 1) (layer "B.Cu") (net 5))
 (segment (start 73.5 57) (end 76.5 57) (width 1) (layer "B.Cu") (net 5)))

